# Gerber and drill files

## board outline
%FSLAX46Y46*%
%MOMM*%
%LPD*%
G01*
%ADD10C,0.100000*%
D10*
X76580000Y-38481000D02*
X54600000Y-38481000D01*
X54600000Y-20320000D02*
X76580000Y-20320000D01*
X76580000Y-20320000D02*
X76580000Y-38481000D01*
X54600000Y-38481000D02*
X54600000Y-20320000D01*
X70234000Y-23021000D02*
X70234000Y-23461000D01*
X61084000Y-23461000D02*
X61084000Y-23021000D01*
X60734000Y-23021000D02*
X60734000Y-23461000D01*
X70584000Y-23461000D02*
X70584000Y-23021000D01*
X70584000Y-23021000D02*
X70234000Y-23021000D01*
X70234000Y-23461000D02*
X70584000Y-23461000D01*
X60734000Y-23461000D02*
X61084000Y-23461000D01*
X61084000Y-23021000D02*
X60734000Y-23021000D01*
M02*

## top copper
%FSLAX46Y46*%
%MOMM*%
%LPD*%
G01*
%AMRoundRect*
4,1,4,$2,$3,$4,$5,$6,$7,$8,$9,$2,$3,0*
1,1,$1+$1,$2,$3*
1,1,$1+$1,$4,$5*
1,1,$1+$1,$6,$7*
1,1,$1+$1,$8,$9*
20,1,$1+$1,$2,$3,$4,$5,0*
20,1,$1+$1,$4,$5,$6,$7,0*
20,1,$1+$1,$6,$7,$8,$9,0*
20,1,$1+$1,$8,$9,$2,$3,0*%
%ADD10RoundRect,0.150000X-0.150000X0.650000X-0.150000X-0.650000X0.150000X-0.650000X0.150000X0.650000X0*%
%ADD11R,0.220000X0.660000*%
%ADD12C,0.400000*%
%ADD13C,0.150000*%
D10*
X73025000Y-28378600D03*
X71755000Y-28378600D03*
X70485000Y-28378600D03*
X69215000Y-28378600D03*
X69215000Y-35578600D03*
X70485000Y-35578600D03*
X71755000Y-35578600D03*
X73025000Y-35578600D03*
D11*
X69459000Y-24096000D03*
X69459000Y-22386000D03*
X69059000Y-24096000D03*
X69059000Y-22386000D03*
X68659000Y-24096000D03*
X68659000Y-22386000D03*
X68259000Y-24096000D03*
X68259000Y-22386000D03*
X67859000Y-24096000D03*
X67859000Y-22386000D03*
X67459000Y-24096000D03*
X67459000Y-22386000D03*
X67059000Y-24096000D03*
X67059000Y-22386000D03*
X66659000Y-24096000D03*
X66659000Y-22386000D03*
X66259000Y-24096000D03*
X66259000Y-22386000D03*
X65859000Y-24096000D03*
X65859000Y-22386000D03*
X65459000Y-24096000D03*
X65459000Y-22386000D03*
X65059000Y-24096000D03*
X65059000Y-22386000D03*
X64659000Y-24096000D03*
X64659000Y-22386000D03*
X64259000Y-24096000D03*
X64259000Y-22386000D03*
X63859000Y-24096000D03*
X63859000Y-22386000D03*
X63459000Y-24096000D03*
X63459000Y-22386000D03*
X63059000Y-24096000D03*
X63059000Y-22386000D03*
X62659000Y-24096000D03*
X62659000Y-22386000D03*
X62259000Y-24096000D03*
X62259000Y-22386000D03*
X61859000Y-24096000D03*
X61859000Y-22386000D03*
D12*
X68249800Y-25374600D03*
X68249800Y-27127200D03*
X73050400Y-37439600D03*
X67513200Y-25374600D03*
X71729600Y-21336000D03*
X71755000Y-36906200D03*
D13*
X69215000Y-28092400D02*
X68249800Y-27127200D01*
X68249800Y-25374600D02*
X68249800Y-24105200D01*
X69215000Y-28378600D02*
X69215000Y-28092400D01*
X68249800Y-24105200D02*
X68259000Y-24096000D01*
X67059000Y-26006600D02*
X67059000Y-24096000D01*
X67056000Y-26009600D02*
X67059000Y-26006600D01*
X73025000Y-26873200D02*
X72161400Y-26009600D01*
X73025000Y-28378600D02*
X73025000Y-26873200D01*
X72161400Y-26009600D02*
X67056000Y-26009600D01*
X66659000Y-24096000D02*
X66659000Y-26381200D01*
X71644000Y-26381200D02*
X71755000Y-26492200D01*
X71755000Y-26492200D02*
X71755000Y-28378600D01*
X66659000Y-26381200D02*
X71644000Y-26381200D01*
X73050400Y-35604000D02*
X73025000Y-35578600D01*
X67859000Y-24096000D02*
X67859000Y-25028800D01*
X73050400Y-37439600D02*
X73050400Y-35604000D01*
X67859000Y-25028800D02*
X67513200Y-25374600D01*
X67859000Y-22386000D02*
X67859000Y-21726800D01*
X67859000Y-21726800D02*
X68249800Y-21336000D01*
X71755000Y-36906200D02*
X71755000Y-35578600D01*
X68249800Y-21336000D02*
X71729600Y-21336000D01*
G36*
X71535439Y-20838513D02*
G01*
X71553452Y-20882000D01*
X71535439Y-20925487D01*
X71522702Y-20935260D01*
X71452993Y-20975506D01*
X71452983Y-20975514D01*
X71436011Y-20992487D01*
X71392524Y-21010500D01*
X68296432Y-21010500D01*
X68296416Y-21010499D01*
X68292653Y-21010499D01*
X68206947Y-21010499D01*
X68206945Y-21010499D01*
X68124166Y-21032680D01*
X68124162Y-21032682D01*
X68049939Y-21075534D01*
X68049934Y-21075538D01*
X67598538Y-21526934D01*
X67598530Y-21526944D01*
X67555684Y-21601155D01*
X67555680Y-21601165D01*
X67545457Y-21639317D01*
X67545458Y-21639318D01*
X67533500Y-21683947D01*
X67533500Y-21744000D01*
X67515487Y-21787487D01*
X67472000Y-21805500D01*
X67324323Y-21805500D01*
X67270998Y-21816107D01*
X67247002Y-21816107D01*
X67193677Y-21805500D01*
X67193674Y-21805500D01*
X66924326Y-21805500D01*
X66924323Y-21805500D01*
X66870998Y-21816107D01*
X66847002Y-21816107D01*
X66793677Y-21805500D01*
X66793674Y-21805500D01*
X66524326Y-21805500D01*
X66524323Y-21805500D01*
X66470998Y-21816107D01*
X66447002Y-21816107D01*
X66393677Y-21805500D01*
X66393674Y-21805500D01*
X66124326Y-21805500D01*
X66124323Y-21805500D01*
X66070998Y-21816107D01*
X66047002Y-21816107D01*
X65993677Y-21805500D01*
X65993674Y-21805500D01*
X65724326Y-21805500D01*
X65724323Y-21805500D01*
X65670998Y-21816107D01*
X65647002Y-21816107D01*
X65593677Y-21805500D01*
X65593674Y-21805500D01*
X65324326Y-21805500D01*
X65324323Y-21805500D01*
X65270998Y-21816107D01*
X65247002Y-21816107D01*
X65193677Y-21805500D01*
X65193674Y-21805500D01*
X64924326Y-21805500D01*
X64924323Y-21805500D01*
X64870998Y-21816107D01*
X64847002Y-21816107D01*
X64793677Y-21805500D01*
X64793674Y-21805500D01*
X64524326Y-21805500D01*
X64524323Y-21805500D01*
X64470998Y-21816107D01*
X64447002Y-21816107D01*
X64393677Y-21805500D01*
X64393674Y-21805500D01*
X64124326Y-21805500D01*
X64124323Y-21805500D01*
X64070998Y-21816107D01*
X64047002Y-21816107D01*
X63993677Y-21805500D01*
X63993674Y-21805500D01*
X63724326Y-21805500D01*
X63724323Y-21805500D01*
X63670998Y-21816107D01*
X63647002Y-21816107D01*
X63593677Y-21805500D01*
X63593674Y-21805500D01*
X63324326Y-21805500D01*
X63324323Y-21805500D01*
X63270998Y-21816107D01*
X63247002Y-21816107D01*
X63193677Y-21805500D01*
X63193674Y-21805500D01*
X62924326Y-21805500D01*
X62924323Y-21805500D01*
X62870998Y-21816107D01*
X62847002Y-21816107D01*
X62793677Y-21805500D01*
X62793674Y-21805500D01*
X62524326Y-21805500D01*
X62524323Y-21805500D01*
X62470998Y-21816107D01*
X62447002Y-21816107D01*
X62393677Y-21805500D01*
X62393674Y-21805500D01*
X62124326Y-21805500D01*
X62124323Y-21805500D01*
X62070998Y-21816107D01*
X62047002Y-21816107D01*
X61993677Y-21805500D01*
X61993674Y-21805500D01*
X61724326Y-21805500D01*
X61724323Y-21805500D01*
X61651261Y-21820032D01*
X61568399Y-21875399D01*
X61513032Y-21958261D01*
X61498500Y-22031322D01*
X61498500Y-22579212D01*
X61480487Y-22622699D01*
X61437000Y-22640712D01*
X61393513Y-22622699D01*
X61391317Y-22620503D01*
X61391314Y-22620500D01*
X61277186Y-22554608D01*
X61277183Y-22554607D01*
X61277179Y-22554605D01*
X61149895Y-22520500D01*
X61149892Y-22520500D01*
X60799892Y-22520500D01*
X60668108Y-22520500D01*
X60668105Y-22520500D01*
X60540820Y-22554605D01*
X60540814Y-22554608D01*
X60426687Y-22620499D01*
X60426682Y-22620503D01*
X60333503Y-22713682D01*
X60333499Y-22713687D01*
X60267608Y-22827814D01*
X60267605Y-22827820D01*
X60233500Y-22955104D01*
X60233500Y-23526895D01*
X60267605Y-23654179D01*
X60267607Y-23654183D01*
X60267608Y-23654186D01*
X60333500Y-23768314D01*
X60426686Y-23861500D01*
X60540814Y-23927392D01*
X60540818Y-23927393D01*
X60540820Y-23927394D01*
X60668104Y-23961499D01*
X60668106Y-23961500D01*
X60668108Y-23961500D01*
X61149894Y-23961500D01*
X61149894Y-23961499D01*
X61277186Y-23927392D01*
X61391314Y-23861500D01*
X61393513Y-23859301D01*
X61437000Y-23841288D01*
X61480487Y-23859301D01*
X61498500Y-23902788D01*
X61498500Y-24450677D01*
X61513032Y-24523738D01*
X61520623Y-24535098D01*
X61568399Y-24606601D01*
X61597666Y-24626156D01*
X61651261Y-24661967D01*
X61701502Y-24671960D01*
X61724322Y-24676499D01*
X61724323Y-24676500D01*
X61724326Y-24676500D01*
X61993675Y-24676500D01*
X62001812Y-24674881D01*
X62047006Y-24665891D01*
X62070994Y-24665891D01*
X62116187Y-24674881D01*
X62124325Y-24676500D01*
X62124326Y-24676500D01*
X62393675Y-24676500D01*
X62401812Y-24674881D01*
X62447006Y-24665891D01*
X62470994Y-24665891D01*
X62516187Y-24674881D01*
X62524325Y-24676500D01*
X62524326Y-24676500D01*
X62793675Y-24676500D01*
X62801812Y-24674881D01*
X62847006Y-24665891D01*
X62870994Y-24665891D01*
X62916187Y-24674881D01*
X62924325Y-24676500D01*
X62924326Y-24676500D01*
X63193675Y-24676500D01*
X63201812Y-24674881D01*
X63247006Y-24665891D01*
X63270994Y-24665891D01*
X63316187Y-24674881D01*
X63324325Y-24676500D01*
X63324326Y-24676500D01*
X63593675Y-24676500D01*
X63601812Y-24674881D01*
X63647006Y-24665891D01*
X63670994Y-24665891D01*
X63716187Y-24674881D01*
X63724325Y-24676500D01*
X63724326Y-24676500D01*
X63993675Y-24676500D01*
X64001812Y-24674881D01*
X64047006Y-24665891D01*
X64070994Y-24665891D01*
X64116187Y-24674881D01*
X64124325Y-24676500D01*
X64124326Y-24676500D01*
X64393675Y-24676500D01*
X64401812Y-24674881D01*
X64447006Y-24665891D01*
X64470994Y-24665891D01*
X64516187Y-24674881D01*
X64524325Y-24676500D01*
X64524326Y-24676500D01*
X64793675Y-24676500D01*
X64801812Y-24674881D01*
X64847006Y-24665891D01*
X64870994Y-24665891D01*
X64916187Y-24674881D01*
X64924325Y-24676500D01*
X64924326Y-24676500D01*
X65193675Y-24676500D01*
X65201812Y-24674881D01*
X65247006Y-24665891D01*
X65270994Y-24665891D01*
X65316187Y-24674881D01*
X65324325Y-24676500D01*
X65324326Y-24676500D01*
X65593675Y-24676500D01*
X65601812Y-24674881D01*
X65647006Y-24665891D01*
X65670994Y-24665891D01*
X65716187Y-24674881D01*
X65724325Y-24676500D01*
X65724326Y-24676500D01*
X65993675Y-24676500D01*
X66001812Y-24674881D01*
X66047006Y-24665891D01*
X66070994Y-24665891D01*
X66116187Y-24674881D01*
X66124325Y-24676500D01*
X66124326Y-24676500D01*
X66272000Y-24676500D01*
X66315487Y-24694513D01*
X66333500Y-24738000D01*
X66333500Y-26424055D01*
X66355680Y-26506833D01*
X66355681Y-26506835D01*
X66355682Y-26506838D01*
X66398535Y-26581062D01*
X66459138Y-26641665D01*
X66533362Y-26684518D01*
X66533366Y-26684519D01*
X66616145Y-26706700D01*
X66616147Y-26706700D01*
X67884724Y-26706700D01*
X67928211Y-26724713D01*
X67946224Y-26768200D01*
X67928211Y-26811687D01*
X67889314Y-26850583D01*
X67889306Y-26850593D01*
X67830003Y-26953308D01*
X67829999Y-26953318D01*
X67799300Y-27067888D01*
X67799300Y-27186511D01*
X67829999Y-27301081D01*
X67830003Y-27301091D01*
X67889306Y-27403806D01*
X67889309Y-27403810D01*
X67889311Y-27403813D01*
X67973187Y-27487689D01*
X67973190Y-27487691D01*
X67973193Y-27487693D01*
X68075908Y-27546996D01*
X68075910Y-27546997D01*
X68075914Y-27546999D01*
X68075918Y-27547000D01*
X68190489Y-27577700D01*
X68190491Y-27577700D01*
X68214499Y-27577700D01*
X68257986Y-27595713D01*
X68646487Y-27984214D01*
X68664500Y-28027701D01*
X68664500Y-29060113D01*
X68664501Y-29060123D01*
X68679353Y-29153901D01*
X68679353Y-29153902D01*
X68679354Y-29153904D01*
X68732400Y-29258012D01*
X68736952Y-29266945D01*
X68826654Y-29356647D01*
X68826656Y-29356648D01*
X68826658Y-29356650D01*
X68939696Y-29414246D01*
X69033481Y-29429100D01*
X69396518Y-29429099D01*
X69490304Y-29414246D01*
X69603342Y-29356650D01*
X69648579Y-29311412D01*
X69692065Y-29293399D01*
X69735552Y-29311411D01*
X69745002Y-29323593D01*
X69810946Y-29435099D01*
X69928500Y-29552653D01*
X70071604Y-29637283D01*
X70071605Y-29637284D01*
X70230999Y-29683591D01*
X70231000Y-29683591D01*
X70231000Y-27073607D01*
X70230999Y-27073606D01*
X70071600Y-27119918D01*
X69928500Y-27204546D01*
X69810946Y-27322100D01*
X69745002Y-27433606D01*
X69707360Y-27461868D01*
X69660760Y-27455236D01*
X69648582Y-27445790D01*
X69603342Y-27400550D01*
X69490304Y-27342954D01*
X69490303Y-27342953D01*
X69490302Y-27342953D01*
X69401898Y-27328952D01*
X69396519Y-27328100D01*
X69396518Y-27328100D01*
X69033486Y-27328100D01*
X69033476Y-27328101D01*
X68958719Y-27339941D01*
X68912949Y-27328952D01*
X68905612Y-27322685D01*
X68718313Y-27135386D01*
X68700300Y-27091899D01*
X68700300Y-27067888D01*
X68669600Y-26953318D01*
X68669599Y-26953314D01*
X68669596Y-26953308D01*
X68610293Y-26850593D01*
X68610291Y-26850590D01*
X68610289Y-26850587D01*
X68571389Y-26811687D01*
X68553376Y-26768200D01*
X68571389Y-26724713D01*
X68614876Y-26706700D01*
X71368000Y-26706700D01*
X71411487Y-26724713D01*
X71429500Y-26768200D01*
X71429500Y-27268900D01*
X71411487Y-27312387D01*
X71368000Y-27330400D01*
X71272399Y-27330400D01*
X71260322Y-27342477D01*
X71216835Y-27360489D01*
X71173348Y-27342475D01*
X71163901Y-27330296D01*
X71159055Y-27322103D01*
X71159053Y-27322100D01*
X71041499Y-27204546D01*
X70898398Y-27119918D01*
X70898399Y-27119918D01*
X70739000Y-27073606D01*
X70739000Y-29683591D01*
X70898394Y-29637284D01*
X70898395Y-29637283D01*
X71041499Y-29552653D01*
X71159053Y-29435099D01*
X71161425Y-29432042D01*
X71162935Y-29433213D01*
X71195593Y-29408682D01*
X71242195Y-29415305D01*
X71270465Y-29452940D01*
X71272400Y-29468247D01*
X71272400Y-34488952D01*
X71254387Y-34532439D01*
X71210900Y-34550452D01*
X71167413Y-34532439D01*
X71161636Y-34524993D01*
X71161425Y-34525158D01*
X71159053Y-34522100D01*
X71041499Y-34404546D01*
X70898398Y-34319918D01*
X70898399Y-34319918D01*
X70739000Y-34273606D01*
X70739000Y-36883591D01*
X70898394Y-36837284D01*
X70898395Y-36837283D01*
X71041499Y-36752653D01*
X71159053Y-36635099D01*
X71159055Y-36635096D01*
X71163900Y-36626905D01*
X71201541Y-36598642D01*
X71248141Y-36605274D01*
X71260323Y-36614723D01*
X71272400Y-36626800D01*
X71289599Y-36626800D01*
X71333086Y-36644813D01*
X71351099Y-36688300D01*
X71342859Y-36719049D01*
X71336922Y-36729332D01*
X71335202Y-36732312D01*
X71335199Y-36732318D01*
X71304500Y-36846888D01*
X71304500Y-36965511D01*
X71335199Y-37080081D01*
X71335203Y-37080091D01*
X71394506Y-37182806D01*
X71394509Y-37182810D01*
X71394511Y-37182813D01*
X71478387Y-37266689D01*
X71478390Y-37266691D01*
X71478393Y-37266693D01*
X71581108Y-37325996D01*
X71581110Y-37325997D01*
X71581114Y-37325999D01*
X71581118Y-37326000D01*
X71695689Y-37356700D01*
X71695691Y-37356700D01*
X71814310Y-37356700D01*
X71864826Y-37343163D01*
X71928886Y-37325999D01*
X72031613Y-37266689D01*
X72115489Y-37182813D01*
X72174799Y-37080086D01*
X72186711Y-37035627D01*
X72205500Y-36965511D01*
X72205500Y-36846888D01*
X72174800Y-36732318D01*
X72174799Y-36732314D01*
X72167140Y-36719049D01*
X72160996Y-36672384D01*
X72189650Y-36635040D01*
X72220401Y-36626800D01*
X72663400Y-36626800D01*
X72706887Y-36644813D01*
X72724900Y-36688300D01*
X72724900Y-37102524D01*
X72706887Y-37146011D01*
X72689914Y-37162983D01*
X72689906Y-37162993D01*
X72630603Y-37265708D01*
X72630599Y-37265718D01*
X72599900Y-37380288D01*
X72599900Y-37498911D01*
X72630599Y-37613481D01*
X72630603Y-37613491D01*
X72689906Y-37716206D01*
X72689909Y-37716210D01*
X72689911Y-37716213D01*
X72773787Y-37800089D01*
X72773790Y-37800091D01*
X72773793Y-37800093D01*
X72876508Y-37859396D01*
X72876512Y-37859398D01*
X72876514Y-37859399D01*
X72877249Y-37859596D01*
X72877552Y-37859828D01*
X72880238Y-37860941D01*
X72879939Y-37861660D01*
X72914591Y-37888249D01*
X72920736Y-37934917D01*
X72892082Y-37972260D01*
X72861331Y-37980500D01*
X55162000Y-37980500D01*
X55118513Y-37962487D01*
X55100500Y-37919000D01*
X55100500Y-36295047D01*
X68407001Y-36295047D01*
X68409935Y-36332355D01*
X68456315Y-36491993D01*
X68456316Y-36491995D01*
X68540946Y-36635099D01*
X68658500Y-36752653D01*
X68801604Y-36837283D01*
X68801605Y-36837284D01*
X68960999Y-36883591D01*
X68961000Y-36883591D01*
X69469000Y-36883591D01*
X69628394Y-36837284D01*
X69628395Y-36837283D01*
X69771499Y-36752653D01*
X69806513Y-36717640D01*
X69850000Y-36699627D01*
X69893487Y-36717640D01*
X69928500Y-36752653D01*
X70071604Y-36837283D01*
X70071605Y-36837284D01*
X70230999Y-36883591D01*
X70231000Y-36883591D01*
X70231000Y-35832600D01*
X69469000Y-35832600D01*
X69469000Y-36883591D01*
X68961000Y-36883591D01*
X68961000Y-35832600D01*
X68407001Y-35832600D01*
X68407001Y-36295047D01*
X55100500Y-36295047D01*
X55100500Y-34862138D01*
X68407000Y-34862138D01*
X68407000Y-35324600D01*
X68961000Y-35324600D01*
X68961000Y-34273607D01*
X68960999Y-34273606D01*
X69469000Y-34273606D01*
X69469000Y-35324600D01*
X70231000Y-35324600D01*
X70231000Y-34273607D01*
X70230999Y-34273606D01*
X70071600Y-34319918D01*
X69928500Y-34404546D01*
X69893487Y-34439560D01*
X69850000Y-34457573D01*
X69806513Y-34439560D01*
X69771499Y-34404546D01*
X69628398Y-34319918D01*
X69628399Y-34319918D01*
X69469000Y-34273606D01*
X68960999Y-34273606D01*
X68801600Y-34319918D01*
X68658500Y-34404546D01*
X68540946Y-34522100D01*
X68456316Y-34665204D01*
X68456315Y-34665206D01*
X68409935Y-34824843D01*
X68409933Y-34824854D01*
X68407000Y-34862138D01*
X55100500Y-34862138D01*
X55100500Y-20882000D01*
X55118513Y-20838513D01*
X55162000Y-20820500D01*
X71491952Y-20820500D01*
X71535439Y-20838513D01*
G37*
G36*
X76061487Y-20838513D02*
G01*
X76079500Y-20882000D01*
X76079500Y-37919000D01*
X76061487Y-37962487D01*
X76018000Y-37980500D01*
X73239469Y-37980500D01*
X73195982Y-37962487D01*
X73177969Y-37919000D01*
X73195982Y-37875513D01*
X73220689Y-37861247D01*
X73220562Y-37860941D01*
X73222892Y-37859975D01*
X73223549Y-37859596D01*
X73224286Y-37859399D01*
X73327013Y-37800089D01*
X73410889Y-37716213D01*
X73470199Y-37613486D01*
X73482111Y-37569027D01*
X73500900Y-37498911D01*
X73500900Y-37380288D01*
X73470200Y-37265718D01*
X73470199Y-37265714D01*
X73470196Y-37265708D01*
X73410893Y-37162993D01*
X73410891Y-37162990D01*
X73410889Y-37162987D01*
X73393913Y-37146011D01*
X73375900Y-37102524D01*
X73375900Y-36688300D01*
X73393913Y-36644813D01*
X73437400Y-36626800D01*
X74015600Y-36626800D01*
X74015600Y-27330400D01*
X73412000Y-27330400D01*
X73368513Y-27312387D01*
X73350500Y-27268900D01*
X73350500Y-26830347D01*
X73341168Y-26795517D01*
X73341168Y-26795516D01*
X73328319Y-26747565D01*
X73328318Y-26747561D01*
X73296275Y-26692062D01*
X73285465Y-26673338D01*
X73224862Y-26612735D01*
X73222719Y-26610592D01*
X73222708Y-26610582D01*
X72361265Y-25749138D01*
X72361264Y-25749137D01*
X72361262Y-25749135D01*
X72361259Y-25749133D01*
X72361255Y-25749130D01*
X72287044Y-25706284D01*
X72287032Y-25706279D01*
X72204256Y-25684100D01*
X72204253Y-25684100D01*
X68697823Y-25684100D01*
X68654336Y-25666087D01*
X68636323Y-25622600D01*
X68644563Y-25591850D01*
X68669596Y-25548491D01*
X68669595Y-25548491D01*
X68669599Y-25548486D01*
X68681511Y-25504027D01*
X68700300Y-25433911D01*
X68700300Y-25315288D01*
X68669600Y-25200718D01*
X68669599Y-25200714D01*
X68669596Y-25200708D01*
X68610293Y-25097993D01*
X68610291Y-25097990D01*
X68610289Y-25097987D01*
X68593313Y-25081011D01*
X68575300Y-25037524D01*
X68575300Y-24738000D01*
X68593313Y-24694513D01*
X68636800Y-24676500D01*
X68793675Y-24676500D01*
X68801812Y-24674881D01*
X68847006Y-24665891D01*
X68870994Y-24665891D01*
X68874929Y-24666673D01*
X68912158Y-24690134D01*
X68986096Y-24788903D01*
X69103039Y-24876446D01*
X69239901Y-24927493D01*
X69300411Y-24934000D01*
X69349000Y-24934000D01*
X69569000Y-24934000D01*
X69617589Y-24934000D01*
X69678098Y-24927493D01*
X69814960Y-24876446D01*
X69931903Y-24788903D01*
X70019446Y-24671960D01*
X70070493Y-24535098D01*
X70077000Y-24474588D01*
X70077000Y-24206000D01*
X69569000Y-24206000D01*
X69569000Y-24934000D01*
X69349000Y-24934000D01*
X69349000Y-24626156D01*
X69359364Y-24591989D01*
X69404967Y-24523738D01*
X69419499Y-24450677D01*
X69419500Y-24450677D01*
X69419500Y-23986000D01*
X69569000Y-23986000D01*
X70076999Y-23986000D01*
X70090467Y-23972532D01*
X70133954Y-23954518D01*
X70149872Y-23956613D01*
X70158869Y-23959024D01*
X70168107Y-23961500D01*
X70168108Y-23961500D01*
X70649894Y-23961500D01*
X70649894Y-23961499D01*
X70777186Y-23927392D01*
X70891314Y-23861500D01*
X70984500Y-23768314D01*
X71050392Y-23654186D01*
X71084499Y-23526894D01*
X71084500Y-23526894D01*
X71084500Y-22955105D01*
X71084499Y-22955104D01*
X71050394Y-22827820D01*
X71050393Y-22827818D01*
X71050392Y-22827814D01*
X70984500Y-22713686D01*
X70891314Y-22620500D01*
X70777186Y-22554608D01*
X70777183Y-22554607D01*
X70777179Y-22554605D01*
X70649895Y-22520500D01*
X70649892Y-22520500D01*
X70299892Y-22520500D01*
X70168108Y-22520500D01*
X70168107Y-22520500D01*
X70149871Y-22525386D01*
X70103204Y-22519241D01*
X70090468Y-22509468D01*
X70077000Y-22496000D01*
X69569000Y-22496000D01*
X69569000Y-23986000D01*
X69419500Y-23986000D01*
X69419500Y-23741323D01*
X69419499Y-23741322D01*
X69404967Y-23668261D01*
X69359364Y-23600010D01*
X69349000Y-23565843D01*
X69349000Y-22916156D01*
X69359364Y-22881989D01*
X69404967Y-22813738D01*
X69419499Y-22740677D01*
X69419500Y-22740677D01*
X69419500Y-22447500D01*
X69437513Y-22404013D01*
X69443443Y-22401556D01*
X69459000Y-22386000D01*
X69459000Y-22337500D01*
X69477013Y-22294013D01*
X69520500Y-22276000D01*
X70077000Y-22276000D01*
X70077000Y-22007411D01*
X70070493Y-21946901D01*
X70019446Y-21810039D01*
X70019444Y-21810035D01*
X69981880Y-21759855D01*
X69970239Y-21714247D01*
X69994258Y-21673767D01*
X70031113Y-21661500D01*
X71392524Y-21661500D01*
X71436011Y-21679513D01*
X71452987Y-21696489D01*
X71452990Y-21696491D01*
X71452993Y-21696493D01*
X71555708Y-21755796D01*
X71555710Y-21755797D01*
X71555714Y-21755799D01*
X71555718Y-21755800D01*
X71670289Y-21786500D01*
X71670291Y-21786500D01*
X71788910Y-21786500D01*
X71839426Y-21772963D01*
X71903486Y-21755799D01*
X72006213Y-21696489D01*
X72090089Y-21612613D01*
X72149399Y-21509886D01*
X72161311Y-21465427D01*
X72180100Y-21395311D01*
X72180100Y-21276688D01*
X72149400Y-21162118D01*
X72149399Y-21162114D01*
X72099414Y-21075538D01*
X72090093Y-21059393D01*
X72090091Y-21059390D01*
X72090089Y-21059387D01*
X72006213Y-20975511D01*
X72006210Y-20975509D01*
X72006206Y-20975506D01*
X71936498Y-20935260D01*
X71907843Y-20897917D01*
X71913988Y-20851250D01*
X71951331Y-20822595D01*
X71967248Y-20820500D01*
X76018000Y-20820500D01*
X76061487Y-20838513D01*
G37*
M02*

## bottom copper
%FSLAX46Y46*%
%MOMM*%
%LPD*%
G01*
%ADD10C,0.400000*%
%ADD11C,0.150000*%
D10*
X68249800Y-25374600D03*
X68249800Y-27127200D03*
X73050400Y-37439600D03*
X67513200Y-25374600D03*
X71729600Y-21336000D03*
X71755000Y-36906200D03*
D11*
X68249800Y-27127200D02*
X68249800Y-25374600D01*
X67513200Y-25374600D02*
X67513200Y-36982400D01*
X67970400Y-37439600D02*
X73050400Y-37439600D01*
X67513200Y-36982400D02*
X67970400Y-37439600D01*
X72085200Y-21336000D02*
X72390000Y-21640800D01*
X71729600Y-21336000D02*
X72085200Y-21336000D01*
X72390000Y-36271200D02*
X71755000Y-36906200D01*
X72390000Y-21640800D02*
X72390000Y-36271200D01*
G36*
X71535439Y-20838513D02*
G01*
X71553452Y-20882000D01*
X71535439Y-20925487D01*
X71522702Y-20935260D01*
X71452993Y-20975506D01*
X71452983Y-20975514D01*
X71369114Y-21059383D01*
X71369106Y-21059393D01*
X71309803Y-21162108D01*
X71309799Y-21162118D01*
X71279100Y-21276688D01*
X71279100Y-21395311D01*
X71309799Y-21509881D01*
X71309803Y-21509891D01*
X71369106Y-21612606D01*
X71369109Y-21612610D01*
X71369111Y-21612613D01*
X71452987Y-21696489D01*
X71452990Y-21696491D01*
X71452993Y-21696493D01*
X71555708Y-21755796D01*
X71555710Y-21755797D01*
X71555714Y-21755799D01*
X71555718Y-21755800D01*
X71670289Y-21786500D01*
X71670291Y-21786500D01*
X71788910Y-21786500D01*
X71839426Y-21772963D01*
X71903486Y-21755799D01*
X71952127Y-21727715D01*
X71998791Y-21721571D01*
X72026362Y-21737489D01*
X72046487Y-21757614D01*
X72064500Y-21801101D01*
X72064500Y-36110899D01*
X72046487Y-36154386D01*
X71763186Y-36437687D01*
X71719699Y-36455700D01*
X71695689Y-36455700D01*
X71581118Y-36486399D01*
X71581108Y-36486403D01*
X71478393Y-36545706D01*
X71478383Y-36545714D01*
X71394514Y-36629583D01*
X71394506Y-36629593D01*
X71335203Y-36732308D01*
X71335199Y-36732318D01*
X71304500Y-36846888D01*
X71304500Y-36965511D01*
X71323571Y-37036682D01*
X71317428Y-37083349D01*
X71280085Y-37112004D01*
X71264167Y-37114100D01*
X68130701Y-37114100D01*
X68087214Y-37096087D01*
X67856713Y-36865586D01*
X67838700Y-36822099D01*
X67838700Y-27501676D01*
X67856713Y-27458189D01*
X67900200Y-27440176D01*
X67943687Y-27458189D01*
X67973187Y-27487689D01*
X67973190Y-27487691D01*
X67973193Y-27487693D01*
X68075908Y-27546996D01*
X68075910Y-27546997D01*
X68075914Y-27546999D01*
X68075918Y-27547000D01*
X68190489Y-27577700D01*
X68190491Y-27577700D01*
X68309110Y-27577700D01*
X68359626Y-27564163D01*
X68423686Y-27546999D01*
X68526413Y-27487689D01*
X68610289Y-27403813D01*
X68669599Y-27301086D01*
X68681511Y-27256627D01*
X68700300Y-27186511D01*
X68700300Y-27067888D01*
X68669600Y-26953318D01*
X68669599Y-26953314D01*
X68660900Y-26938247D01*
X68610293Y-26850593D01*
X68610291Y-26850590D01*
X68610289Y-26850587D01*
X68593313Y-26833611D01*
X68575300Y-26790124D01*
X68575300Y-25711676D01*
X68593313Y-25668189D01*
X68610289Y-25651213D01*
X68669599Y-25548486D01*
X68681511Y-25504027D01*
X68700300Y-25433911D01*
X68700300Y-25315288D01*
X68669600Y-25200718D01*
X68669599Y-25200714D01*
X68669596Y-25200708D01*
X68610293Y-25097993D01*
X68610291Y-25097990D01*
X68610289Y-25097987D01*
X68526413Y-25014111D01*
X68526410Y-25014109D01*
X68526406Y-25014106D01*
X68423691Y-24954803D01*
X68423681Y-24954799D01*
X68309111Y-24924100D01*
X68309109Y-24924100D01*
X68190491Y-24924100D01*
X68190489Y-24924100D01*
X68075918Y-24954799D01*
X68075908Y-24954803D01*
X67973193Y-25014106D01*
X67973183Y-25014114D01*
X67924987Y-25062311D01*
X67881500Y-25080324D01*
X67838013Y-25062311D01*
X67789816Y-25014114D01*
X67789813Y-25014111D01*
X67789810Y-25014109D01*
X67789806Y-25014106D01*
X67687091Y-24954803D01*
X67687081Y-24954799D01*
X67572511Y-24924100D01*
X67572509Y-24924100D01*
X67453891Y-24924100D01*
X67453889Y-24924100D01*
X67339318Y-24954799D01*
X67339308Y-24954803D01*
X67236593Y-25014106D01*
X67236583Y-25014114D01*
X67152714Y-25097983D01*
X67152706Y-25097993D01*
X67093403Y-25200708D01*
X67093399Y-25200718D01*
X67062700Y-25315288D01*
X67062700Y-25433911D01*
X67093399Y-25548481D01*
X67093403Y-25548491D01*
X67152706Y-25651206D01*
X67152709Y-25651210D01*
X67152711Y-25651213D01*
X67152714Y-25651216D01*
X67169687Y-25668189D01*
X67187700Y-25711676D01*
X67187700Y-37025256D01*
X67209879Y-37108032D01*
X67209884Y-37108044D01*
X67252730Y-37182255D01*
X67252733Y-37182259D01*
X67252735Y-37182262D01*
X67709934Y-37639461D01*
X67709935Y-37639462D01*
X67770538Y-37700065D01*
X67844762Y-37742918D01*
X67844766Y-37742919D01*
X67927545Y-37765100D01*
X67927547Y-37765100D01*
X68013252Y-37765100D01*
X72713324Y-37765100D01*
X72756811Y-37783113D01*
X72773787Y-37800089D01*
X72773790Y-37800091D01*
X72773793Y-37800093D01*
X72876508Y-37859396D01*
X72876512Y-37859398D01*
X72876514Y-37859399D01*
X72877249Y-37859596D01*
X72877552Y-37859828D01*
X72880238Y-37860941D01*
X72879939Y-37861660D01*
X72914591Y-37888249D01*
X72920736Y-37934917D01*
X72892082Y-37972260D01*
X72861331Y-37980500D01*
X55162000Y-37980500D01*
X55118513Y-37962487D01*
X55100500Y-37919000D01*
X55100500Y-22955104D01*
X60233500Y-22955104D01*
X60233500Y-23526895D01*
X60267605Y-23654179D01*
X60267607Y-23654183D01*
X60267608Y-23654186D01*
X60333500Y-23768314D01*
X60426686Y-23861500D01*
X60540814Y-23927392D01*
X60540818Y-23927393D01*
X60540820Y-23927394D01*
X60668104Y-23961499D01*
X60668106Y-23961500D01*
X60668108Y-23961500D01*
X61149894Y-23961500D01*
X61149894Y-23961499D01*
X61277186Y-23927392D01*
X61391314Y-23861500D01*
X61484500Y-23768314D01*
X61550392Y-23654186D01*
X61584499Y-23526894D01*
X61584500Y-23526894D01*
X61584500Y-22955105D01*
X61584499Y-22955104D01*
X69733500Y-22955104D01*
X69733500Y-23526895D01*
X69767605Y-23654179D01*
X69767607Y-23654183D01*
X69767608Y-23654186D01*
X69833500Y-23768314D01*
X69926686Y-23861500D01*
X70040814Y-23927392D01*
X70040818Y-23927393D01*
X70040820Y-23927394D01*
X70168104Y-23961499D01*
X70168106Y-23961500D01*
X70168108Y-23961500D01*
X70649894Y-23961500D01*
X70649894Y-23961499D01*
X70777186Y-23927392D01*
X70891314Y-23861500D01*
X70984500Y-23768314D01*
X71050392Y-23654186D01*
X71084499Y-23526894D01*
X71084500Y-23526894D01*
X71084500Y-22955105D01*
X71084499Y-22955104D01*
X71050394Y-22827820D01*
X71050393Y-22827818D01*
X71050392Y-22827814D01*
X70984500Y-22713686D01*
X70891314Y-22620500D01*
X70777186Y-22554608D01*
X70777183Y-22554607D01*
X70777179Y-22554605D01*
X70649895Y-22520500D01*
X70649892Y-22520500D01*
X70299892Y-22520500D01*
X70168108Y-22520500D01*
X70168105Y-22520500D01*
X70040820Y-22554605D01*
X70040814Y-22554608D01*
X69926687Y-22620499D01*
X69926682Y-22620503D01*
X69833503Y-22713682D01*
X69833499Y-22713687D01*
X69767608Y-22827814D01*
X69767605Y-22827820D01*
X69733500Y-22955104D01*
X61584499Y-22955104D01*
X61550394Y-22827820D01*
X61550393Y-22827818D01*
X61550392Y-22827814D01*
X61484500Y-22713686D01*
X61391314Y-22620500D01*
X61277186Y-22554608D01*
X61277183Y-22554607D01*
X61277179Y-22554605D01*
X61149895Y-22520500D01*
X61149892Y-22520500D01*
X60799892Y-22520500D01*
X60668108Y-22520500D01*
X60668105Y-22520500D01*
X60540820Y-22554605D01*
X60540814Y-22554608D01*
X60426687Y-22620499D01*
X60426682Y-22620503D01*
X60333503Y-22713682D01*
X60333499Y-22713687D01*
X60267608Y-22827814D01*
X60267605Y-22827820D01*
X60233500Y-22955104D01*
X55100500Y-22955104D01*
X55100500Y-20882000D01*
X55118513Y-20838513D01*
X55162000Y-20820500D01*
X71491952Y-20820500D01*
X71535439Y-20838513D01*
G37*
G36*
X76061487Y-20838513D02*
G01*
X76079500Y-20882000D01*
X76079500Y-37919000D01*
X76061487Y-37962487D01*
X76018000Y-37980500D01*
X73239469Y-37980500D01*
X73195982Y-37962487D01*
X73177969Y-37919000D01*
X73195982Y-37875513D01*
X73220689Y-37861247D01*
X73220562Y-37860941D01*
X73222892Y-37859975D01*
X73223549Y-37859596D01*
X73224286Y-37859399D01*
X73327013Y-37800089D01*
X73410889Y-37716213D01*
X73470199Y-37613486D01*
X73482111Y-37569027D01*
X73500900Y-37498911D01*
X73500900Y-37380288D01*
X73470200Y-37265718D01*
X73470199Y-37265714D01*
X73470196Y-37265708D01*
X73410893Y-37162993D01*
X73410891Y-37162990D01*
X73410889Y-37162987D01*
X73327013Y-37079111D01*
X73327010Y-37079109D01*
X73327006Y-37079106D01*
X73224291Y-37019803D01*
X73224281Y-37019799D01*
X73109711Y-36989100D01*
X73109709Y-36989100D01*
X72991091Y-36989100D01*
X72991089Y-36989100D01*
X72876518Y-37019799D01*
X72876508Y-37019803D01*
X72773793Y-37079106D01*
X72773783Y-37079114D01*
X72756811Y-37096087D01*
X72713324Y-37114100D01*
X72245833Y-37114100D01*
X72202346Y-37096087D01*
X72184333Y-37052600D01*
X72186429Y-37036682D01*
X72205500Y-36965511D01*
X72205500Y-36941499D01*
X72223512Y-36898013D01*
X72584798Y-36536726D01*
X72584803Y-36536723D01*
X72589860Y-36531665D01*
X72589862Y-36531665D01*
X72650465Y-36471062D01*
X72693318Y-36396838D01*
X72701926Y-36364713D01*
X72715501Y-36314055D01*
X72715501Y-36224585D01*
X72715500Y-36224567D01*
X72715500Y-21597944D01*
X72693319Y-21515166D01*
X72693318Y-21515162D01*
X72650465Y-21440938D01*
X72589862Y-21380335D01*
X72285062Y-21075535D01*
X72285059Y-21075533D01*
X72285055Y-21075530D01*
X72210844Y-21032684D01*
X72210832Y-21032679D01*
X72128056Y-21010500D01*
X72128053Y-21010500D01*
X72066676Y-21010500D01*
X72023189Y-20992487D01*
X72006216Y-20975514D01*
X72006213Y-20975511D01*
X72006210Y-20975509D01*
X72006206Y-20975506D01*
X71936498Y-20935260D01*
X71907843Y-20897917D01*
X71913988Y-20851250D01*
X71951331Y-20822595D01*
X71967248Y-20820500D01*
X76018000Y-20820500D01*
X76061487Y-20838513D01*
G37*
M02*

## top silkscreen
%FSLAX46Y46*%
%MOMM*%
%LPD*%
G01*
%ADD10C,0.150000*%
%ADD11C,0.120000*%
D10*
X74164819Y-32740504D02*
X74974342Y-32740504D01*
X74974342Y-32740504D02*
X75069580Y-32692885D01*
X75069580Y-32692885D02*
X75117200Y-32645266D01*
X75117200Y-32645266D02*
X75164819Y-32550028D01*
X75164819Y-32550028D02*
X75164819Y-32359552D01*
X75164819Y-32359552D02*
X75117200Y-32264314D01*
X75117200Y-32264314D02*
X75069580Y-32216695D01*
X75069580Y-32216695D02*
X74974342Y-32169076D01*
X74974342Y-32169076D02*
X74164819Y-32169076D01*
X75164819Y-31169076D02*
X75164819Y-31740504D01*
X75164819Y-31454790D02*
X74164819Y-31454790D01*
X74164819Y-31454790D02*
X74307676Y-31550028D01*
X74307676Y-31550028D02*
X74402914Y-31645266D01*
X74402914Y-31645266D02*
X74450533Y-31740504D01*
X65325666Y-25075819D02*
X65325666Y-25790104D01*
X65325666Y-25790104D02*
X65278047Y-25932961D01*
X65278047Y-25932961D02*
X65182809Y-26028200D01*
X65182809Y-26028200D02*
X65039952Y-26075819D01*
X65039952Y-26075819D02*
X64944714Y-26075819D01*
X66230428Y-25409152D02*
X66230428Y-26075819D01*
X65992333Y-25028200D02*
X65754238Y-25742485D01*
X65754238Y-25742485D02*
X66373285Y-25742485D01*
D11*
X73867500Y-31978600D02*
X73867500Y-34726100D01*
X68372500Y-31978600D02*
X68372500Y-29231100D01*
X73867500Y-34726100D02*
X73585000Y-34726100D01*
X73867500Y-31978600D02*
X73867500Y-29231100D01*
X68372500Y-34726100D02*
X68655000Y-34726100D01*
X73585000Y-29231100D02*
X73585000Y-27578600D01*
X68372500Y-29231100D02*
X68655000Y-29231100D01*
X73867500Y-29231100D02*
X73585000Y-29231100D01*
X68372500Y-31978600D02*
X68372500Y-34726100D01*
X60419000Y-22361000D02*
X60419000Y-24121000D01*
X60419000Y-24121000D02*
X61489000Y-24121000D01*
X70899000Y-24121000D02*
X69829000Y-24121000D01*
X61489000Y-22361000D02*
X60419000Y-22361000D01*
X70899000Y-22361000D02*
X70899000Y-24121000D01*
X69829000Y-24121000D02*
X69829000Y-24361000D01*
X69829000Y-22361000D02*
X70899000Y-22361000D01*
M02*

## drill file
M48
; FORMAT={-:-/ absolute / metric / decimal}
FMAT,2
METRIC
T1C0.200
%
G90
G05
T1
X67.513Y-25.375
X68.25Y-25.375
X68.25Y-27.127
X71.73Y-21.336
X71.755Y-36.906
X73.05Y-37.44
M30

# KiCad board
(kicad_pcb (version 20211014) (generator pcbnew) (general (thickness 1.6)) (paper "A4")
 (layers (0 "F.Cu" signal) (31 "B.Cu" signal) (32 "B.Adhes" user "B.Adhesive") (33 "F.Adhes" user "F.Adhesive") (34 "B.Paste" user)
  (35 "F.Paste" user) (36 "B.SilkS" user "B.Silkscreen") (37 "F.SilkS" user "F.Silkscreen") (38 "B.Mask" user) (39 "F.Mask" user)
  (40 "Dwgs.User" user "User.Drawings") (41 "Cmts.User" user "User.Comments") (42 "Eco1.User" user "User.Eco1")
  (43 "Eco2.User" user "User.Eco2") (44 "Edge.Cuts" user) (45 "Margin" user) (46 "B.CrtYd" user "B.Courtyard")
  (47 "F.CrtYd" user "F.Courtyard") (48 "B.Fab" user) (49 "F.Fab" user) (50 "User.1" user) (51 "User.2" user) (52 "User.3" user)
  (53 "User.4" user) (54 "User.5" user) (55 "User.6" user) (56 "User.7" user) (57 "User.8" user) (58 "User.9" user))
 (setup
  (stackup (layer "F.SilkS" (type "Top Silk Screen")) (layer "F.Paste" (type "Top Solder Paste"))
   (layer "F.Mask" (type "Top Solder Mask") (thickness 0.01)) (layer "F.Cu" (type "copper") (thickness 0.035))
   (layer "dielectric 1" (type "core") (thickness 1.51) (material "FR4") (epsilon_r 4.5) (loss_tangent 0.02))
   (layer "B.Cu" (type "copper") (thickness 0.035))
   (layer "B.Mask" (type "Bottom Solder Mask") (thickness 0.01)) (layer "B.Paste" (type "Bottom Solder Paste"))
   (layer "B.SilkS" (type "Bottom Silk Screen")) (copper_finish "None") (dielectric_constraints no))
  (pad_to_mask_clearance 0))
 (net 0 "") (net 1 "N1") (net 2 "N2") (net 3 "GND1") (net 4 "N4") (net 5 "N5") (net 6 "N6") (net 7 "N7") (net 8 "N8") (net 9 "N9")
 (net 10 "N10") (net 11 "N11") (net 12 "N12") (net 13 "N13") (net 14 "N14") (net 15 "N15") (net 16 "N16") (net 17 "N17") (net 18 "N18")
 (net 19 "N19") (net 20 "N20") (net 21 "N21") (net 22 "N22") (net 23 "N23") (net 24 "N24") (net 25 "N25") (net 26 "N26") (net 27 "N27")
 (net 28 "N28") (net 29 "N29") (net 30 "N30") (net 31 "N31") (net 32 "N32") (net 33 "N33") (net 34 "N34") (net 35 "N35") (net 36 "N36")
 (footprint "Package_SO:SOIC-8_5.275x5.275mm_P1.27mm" (layer "F.Cu") (at 71.12 31.9786 -90)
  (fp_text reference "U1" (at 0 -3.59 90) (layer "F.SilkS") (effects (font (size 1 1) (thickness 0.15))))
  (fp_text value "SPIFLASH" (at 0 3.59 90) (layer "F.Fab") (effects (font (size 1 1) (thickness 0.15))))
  (fp_line (start 0 -2.7475) (end 2.7475 -2.7475) (layer "F.SilkS") (width 0.12))
  (fp_line (start 0 2.7475) (end -2.7475 2.7475) (layer "F.SilkS") (width 0.12))
  (fp_line (start 2.7475 -2.7475) (end 2.7475 -2.465) (layer "F.SilkS") (width 0.12))
  (fp_line (start 0 -2.7475) (end -2.7475 -2.7475) (layer "F.SilkS") (width 0.12))
  (fp_line (start 2.7475 2.7475) (end 2.7475 2.465) (layer "F.SilkS") (width 0.12))
  (fp_line (start -2.7475 -2.465) (end -4.4 -2.465) (layer "F.SilkS") (width 0.12))
  (fp_line (start -2.7475 2.7475) (end -2.7475 2.465) (layer "F.SilkS") (width 0.12))
  (fp_line (start -2.7475 -2.7475) (end -2.7475 -2.465) (layer "F.SilkS") (width 0.12))
  (fp_line (start 0 2.7475) (end 2.7475 2.7475) (layer "F.SilkS") (width 0.12))
  (pad "1" smd roundrect (at -3.6 -1.905 270) (size 1.6 0.6) (layers "F.Cu" "F.Paste" "F.Mask") (roundrect_rratio 0.25) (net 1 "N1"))
  (pad "2" smd roundrect (at -3.6 -0.635 270) (size 1.6 0.6) (layers "F.Cu" "F.Paste" "F.Mask") (roundrect_rratio 0.25) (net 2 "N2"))
  (pad "3" smd roundrect (at -3.6 0.635 270) (size 1.6 0.6) (layers "F.Cu" "F.Paste" "F.Mask") (roundrect_rratio 0.25) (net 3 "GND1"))
  (pad "4" smd roundrect (at -3.6 1.905 270) (size 1.6 0.6) (layers "F.Cu" "F.Paste" "F.Mask") (roundrect_rratio 0.25) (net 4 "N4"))
  (pad "5" smd roundrect (at 3.6 1.905 270) (size 1.6 0.6) (layers "F.Cu" "F.Paste" "F.Mask") (roundrect_rratio 0.25) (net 3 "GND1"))
  (pad "6" smd roundrect (at 3.6 0.635 270) (size 1.6 0.6) (layers "F.Cu" "F.Paste" "F.Mask") (roundrect_rratio 0.25) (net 3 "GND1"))
  (pad "7" smd roundrect (at 3.6 -0.635 270) (size 1.6 0.6) (layers "F.Cu" "F.Paste" "F.Mask") (roundrect_rratio 0.25) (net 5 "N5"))
  (pad "8" smd roundrect (at 3.6 -1.905 270) (size 1.6 0.6) (layers "F.Cu" "F.Paste" "F.Mask") (roundrect_rratio 0.25) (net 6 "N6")))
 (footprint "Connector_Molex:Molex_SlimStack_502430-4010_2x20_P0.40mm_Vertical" (layer "F.Cu") (at 65.659 23.241 180)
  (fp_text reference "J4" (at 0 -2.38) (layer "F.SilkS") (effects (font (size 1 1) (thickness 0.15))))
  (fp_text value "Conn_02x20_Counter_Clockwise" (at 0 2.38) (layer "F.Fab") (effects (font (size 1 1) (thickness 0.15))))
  (fp_line (start 5.24 0.88) (end 5.24 -0.88) (layer "F.SilkS") (width 0.12))
  (fp_line (start 5.24 -0.88) (end 4.17 -0.88) (layer "F.SilkS") (width 0.12))
  (fp_line (start -5.24 -0.88) (end -4.17 -0.88) (layer "F.SilkS") (width 0.12))
  (fp_line (start 4.17 0.88) (end 5.24 0.88) (layer "F.SilkS") (width 0.12))
  (fp_line (start -5.24 0.88) (end -5.24 -0.88) (layer "F.SilkS") (width 0.12))
  (fp_line (start -4.17 -0.88) (end -4.17 -1.12) (layer "F.SilkS") (width 0.12))
  (fp_line (start -4.17 0.88) (end -5.24 0.88) (layer "F.SilkS") (width 0.12))
  (fp_line (start -4.575 0.22) (end -4.575 -0.22) (layer "Edge.Cuts") (width 0.1))
  (fp_line (start 4.575 -0.22) (end 4.575 0.22) (layer "Edge.Cuts") (width 0.1))
  (fp_line (start 4.925 0.22) (end 4.925 -0.22) (layer "Edge.Cuts") (width 0.1))
  (fp_line (start -4.925 -0.22) (end -4.925 0.22) (layer "Edge.Cuts") (width 0.1))
  (fp_line (start -4.925 0.22) (end -4.575 0.22) (layer "Edge.Cuts") (width 0.1))
  (fp_line (start -4.575 -0.22) (end -4.925 -0.22) (layer "Edge.Cuts") (width 0.1))
  (fp_line (start 4.925 -0.22) (end 4.575 -0.22) (layer "Edge.Cuts") (width 0.1))
  (fp_line (start 4.575 0.22) (end 4.925 0.22) (layer "Edge.Cuts") (width 0.1))
  (pad "1" smd rect (at -3.8 -0.855 180) (size 0.22 0.66) (layers "F.Cu" "F.Paste" "F.Mask") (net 3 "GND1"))
  (pad "2" smd rect (at -3.8 0.855 180) (size 0.22 0.66) (layers "F.Cu" "F.Paste" "F.Mask") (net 3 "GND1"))
  (pad "3" smd rect (at -3.4 -0.855 180) (size 0.22 0.66) (layers "F.Cu" "F.Paste" "F.Mask") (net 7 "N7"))
  (pad "4" smd rect (at -3.4 0.855 180) (size 0.22 0.66) (layers "F.Cu" "F.Paste" "F.Mask") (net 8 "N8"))
  (pad "5" smd rect (at -3 -0.855 180) (size 0.22 0.66) (layers "F.Cu" "F.Paste" "F.Mask") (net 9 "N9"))
  (pad "6" smd rect (at -3 0.855 180) (size 0.22 0.66) (layers "F.Cu" "F.Paste" "F.Mask") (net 4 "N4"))
  (pad "7" smd rect (at -2.6 -0.855 180) (size 0.22 0.66) (layers "F.Cu" "F.Paste" "F.Mask") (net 4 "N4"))
  (pad "8" smd rect (at -2.6 0.855 180) (size 0.22 0.66) (layers "F.Cu" "F.Paste" "F.Mask") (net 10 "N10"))
  (pad "9" smd rect (at -2.2 -0.855 180) (size 0.22 0.66) (layers "F.Cu" "F.Paste" "F.Mask") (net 6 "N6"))
  (pad "10" smd rect (at -2.2 0.855 180) (size 0.22 0.66) (layers "F.Cu" "F.Paste" "F.Mask") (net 5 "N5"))
  (pad "11" smd rect (at -1.8 -0.855 180) (size 0.22 0.66) (layers "F.Cu" "F.Paste" "F.Mask") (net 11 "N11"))
  (pad "12" smd rect (at -1.8 0.855 180) (size 0.22 0.66) (layers "F.Cu" "F.Paste" "F.Mask") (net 1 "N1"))
  (pad "13" smd rect (at -1.4 -0.855 180) (size 0.22 0.66) (layers "F.Cu" "F.Paste" "F.Mask") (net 1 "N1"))
  (pad "14" smd rect (at -1.4 0.855 180) (size 0.22 0.66) (layers "F.Cu" "F.Paste" "F.Mask") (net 2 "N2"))
  (pad "15" smd rect (at -1 -0.855 180) (size 0.22 0.66) (layers "F.Cu" "F.Paste" "F.Mask") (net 2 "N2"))
  (pad "16" smd rect (at -1 0.855 180) (size 0.22 0.66) (layers "F.Cu" "F.Paste" "F.Mask") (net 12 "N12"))
  (pad "17" smd rect (at -0.6 -0.855 180) (size 0.22 0.66) (layers "F.Cu" "F.Paste" "F.Mask") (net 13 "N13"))
  (pad "18" smd rect (at -0.6 0.855 180) (size 0.22 0.66) (layers "F.Cu" "F.Paste" "F.Mask") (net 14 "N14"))
  (pad "19" smd rect (at -0.2 -0.855 180) (size 0.22 0.66) (layers "F.Cu" "F.Paste" "F.Mask") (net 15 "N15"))
  (pad "20" smd rect (at -0.2 0.855 180) (size 0.22 0.66) (layers "F.Cu" "F.Paste" "F.Mask") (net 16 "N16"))
  (pad "21" smd rect (at 0.2 -0.855 180) (size 0.22 0.66) (layers "F.Cu" "F.Paste" "F.Mask") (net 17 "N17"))
  (pad "22" smd rect (at 0.2 0.855 180) (size 0.22 0.66) (layers "F.Cu" "F.Paste" "F.Mask") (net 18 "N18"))
  (pad "23" smd rect (at 0.6 -0.855 180) (size 0.22 0.66) (layers "F.Cu" "F.Paste" "F.Mask") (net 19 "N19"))
  (pad "24" smd rect (at 0.6 0.855 180) (size 0.22 0.66) (layers "F.Cu" "F.Paste" "F.Mask") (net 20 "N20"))
  (pad "25" smd rect (at 1 -0.855 180) (size 0.22 0.66) (layers "F.Cu" "F.Paste" "F.Mask") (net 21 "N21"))
  (pad "26" smd rect (at 1 0.855 180) (size 0.22 0.66) (layers "F.Cu" "F.Paste" "F.Mask") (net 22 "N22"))
  (pad "27" smd rect (at 1.4 -0.855 180) (size 0.22 0.66) (layers "F.Cu" "F.Paste" "F.Mask") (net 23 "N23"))
  (pad "28" smd rect (at 1.4 0.855 180) (size 0.22 0.66) (layers "F.Cu" "F.Paste" "F.Mask") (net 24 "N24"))
  (pad "29" smd rect (at 1.8 -0.855 180) (size 0.22 0.66) (layers "F.Cu" "F.Paste" "F.Mask") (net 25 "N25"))
  (pad "30" smd rect (at 1.8 0.855 180) (size 0.22 0.66) (layers "F.Cu" "F.Paste" "F.Mask") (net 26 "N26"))
  (pad "31" smd rect (at 2.2 -0.855 180) (size 0.22 0.66) (layers "F.Cu" "F.Paste" "F.Mask") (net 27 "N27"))
  (pad "32" smd rect (at 2.2 0.855 180) (size 0.22 0.66) (layers "F.Cu" "F.Paste" "F.Mask") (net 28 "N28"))
  (pad "33" smd rect (at 2.6 -0.855 180) (size 0.22 0.66) (layers "F.Cu" "F.Paste" "F.Mask") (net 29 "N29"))
  (pad "34" smd rect (at 2.6 0.855 180) (size 0.22 0.66) (layers "F.Cu" "F.Paste" "F.Mask") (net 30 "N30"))
  (pad "35" smd rect (at 3 -0.855 180) (size 0.22 0.66) (layers "F.Cu" "F.Paste" "F.Mask") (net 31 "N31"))
  (pad "36" smd rect (at 3 0.855 180) (size 0.22 0.66) (layers "F.Cu" "F.Paste" "F.Mask") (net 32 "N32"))
  (pad "37" smd rect (at 3.4 -0.855 180) (size 0.22 0.66) (layers "F.Cu" "F.Paste" "F.Mask") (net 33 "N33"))
  (pad "38" smd rect (at 3.4 0.855 180) (size 0.22 0.66) (layers "F.Cu" "F.Paste" "F.Mask") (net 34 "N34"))
  (pad "39" smd rect (at 3.8 -0.855 180) (size 0.22 0.66) (layers "F.Cu" "F.Paste" "F.Mask") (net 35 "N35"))
  (pad "40" smd rect (at 3.8 0.855 180) (size 0.22 0.66) (layers "F.Cu" "F.Paste" "F.Mask") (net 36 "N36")))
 (gr_line (start 76.58 38.481) (end 54.6 38.481) (layer "Edge.Cuts") (width 0.1))
 (gr_line (start 54.6 20.32) (end 76.58 20.32) (layer "Edge.Cuts") (width 0.1))
 (gr_line (start 76.58 20.32) (end 76.58 38.481) (layer "Edge.Cuts") (width 0.1))
 (gr_line (start 54.6 38.481) (end 54.6 20.32) (layer "Edge.Cuts") (width 0.1))
 (segment (start 69.215 28.0924) (end 68.2498 27.1272) (width 0.15) (layer "F.Cu") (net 4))
 (segment (start 68.2498 25.3746) (end 68.2498 24.1052) (width 0.15) (layer "F.Cu") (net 4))
 (segment (start 69.215 28.3786) (end 69.215 28.0924) (width 0.15) (layer "F.Cu") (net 4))
 (segment (start 68.2498 24.1052) (end 68.259 24.096) (width 0.15) (layer "F.Cu") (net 4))
 (via (at 68.2498 25.3746) (size 0.4) (drill 0.2) (layers "F.Cu" "B.Cu") (free) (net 4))
 (via (at 68.2498 27.1272) (size 0.4) (drill 0.2) (layers "F.Cu" "B.Cu") (free) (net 4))
 (segment (start 68.2498 27.1272) (end 68.2498 25.3746) (width 0.15) (layer "B.Cu") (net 4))
 (segment (start 67.059 26.0066) (end 67.059 24.096) (width 0.15) (layer "F.Cu") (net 1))
 (segment (start 67.056 26.0096) (end 67.059 26.0066) (width 0.15) (layer "F.Cu") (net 1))
 (segment (start 73.025 26.8732) (end 72.1614 26.0096) (width 0.15) (layer "F.Cu") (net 1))
 (segment (start 73.025 28.3786) (end 73.025 26.8732) (width 0.15) (layer "F.Cu") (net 1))
 (segment (start 72.1614 26.0096) (end 67.056 26.0096) (width 0.15) (layer "F.Cu") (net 1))
 (segment (start 66.659 24.096) (end 66.659 26.3812) (width 0.15) (layer "F.Cu") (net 2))
 (segment (start 71.644 26.3812) (end 71.755 26.4922) (width 0.15) (layer "F.Cu") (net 2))
 (segment (start 71.755 26.4922) (end 71.755 28.3786) (width 0.15) (layer "F.Cu") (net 2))
 (segment (start 66.659 26.3812) (end 71.644 26.3812) (width 0.15) (layer "F.Cu") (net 2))
 (segment (start 73.0504 35.604) (end 73.025 35.5786) (width 0.15) (layer "F.Cu") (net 6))
 (segment (start 67.859 24.096) (end 67.859 25.0288) (width 0.15) (layer "F.Cu") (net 6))
 (segment (start 73.0504 37.4396) (end 73.0504 35.604) (width 0.15) (layer "F.Cu") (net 6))
 (segment (start 67.859 25.0288) (end 67.5132 25.3746) (width 0.15) (layer "F.Cu") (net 6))
 (via (at 73.0504 37.4396) (size 0.4) (drill 0.2) (layers "F.Cu" "B.Cu") (free) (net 6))
 (via (at 67.5132 25.3746) (size 0.4) (drill 0.2) (layers "F.Cu" "B.Cu") (free) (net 6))
 (segment (start 67.5132 25.3746) (end 67.5132 36.9824) (width 0.15) (layer "B.Cu") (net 6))
 (segment (start 67.9704 37.4396) (end 73.0504 37.4396) (width 0.15) (layer "B.Cu") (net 6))
 (segment (start 67.5132 36.9824) (end 67.9704 37.4396) (width 0.15) (layer "B.Cu") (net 6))
 (segment (start 67.859 22.386) (end 67.859 21.7268) (width 0.15) (layer "F.Cu") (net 5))
 (segment (start 67.859 21.7268) (end 68.2498 21.336) (width 0.15) (layer "F.Cu") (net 5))
 (segment (start 71.755 36.9062) (end 71.755 35.5786) (width 0.15) (layer "F.Cu") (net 5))
 (segment (start 68.2498 21.336) (end 71.7296 21.336) (width 0.15) (layer "F.Cu") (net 5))
 (via (at 71.7296 21.336) (size 0.4) (drill 0.2) (layers "F.Cu" "B.Cu") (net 5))
 (via (at 71.755 36.9062) (size 0.4) (drill 0.2) (layers "F.Cu" "B.Cu") (free) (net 5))
 (segment (start 72.0852 21.336) (end 72.39 21.6408) (width 0.15) (layer "B.Cu") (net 5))
 (segment (start 71.7296 21.336) (end 72.0852 21.336) (width 0.15) (layer "B.Cu") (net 5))
 (segment (start 72.39 36.2712) (end 71.755 36.9062) (width 0.15) (layer "B.Cu") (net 5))
 (segment (start 72.39 21.6408) (end 72.39 36.2712) (width 0.15) (layer "B.Cu") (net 5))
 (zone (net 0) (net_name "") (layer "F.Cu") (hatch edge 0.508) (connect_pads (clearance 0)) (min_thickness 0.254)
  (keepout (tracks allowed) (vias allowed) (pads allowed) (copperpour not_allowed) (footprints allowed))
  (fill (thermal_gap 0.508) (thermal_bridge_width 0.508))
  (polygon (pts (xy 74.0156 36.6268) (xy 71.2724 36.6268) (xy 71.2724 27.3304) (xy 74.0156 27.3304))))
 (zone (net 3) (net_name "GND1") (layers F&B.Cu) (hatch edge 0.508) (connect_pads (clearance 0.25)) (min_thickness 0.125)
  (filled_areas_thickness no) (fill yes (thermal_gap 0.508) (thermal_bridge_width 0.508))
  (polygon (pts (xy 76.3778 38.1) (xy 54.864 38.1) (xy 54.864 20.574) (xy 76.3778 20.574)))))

